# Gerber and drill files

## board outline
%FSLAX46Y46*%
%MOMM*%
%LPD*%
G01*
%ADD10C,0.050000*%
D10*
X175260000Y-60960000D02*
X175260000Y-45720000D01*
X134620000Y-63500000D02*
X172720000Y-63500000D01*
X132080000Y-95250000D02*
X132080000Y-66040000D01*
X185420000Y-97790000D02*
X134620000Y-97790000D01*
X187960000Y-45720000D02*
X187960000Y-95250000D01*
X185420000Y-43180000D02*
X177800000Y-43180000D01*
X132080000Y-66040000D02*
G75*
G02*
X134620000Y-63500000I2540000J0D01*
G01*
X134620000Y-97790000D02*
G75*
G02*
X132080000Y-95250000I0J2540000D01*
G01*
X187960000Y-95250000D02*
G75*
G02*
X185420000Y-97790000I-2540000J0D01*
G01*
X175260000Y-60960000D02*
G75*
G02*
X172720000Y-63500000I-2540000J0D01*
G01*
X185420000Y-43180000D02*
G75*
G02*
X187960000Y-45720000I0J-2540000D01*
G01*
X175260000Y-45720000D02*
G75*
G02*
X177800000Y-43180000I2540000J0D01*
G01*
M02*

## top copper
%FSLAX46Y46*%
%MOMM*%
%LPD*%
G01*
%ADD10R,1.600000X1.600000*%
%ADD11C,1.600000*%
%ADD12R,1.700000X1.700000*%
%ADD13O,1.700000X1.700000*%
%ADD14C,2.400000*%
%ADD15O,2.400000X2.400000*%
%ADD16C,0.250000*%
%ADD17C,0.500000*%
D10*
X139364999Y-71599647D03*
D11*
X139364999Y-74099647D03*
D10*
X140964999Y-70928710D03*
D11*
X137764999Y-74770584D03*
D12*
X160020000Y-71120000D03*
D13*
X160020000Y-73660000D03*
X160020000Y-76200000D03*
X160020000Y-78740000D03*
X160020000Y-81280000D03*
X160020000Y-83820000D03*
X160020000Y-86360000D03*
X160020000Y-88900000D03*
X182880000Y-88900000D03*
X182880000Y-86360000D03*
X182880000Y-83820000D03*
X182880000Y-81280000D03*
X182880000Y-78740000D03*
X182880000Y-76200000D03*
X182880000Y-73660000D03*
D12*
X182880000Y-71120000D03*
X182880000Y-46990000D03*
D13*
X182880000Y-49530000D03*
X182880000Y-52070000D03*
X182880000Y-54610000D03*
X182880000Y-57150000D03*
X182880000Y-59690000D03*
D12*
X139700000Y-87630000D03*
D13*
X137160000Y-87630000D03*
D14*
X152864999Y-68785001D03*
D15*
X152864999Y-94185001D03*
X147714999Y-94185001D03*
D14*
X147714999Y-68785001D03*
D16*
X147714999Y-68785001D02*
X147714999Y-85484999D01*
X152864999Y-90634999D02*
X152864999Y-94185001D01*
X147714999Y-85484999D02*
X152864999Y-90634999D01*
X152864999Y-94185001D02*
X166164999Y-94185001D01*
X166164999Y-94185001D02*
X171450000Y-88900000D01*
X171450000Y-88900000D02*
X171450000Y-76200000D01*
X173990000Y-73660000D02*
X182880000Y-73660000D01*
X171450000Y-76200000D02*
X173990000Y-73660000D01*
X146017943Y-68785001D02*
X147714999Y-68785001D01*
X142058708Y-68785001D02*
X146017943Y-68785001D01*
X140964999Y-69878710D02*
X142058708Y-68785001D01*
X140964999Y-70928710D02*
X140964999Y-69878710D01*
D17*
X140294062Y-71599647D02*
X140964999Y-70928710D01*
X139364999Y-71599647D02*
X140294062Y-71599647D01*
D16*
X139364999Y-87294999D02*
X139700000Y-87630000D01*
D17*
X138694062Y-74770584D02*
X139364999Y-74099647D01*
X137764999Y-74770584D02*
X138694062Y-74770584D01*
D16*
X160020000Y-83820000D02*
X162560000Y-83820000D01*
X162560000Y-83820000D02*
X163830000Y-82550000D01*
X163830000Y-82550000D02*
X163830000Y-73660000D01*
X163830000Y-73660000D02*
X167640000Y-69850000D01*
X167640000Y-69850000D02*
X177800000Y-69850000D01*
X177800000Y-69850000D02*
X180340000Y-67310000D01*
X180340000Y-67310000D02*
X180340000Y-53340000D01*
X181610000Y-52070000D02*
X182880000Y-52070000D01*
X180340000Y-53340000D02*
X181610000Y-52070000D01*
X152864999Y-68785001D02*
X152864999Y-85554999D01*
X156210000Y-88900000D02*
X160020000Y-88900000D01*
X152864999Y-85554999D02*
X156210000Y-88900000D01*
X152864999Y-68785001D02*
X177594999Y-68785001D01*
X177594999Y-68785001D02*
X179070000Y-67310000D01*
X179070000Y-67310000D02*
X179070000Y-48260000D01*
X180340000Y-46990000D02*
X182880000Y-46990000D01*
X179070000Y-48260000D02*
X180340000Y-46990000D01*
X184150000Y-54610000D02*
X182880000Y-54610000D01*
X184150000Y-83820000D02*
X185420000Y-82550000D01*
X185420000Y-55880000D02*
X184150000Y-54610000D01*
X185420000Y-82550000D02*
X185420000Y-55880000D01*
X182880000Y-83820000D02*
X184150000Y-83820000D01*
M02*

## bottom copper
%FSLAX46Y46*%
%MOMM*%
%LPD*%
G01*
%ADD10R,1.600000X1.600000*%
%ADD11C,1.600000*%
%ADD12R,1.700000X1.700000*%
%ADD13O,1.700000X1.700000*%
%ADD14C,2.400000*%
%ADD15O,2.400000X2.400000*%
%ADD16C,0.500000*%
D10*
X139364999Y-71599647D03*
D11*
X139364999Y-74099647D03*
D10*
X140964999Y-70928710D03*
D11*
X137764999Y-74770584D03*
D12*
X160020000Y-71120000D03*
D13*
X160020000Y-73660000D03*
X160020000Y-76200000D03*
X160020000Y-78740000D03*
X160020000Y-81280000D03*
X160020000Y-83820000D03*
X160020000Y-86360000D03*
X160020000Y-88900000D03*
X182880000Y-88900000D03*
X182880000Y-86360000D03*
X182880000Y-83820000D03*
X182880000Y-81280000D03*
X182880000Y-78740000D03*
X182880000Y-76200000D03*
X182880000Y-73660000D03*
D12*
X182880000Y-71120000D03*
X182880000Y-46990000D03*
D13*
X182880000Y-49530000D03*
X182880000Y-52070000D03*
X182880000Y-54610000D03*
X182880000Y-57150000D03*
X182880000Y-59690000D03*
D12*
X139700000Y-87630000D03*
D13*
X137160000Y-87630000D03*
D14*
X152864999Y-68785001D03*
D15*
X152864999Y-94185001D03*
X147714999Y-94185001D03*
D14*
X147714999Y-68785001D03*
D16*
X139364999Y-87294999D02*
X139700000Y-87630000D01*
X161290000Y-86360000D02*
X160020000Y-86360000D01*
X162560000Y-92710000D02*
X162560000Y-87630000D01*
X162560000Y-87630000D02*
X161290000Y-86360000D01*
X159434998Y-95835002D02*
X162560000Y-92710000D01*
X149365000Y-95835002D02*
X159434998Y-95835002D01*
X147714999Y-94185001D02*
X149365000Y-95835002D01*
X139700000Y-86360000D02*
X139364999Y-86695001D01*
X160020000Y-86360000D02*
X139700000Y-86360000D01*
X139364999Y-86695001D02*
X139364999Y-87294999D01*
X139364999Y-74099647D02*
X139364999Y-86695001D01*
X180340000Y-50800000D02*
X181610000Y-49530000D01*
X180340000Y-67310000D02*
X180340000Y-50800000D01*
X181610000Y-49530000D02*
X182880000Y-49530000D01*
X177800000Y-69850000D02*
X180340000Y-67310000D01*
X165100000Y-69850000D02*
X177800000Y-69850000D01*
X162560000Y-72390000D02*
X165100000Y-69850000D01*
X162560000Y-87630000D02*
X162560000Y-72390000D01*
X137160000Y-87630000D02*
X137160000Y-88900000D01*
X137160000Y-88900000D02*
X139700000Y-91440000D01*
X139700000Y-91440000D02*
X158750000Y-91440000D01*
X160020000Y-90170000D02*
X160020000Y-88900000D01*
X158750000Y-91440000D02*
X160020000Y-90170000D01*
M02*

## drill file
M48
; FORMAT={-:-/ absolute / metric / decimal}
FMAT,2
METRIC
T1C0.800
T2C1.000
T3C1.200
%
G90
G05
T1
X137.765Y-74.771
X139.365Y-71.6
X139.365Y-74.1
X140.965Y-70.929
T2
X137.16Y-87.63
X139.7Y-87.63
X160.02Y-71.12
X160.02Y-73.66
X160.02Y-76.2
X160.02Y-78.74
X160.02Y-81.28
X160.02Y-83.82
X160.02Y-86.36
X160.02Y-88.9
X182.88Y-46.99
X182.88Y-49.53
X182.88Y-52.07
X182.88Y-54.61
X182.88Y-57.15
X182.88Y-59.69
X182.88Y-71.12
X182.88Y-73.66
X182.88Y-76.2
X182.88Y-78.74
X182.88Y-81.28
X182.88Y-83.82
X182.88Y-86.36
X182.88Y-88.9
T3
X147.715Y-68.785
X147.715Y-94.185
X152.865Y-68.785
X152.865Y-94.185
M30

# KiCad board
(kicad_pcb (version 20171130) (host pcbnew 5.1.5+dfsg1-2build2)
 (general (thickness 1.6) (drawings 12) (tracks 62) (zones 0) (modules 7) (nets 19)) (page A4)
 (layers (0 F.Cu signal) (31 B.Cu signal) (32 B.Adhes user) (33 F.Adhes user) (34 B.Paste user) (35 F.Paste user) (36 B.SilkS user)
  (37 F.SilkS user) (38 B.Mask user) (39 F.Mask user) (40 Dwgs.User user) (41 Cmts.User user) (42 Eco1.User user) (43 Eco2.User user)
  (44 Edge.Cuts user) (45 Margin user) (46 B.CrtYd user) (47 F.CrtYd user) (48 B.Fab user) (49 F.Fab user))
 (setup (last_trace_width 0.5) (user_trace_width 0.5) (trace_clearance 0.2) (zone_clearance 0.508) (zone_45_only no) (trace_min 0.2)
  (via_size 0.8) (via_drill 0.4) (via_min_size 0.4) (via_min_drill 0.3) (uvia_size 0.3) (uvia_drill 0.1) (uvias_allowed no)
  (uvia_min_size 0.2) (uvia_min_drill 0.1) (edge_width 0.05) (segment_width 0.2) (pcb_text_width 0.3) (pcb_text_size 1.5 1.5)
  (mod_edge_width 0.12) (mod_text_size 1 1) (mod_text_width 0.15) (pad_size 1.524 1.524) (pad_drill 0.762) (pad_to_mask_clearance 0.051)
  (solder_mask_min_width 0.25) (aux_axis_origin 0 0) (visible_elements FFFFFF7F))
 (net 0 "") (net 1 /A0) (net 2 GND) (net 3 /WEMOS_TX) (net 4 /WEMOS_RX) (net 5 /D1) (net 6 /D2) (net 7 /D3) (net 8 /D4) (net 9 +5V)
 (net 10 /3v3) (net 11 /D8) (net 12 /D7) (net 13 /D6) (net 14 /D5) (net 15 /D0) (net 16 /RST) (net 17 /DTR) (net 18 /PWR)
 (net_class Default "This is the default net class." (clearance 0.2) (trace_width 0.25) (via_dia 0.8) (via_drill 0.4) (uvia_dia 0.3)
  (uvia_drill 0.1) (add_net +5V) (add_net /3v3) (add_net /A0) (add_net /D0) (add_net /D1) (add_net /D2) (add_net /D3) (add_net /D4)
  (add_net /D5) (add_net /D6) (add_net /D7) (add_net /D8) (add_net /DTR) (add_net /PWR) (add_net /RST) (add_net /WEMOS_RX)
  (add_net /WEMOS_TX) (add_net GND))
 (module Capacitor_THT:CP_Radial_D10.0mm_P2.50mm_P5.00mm (layer F.Cu) (at 139.364999 71.599647 270)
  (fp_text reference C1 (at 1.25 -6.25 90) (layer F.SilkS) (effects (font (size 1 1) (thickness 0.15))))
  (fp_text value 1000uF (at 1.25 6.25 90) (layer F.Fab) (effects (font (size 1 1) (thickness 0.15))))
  (pad 1 thru_hole rect (at 0 0 270) (size 1.6 1.6) (drill 0.8) (layers *.Cu *.Mask) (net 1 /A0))
  (pad 2 thru_hole circle (at 2.5 0 270) (size 1.6 1.6) (drill 0.8) (layers *.Cu *.Mask) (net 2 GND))
  (pad 1 thru_hole rect (at -0.670937 -1.6 270) (size 1.6 1.6) (drill 0.8) (layers *.Cu *.Mask) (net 1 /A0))
  (pad 2 thru_hole circle (at 3.170937 1.6 270) (size 1.6 1.6) (drill 0.8) (layers *.Cu *.Mask) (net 2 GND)))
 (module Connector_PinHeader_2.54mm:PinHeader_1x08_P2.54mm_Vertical (layer F.Cu) (at 160.02 71.12)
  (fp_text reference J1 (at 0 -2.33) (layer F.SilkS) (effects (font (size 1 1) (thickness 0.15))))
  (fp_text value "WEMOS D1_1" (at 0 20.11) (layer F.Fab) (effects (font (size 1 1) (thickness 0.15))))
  (pad 1 thru_hole rect (at 0 0) (size 1.7 1.7) (drill 1) (layers *.Cu *.Mask) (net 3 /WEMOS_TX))
  (pad 2 thru_hole oval (at 0 2.54) (size 1.7 1.7) (drill 1) (layers *.Cu *.Mask) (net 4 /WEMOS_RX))
  (pad 3 thru_hole oval (at 0 5.08) (size 1.7 1.7) (drill 1) (layers *.Cu *.Mask) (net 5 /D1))
  (pad 4 thru_hole oval (at 0 7.62) (size 1.7 1.7) (drill 1) (layers *.Cu *.Mask) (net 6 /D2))
  (pad 5 thru_hole oval (at 0 10.16) (size 1.7 1.7) (drill 1) (layers *.Cu *.Mask) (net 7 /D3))
  (pad 6 thru_hole oval (at 0 12.7) (size 1.7 1.7) (drill 1) (layers *.Cu *.Mask) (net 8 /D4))
  (pad 7 thru_hole oval (at 0 15.24) (size 1.7 1.7) (drill 1) (layers *.Cu *.Mask) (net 2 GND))
  (pad 8 thru_hole oval (at 0 17.78) (size 1.7 1.7) (drill 1) (layers *.Cu *.Mask) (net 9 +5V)))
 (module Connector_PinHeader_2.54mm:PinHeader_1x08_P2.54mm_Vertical (layer F.Cu) (at 182.88 71.12)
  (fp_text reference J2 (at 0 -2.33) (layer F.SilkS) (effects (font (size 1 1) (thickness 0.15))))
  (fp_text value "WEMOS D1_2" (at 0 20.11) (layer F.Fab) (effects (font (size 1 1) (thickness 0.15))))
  (pad 8 thru_hole oval (at 0 17.78) (size 1.7 1.7) (drill 1) (layers *.Cu *.Mask) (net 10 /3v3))
  (pad 7 thru_hole oval (at 0 15.24) (size 1.7 1.7) (drill 1) (layers *.Cu *.Mask) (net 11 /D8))
  (pad 6 thru_hole oval (at 0 12.7) (size 1.7 1.7) (drill 1) (layers *.Cu *.Mask) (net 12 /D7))
  (pad 5 thru_hole oval (at 0 10.16) (size 1.7 1.7) (drill 1) (layers *.Cu *.Mask) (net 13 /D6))
  (pad 4 thru_hole oval (at 0 7.62) (size 1.7 1.7) (drill 1) (layers *.Cu *.Mask) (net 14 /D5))
  (pad 3 thru_hole oval (at 0 5.08) (size 1.7 1.7) (drill 1) (layers *.Cu *.Mask) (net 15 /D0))
  (pad 2 thru_hole oval (at 0 2.54) (size 1.7 1.7) (drill 1) (layers *.Cu *.Mask) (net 1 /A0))
  (pad 1 thru_hole rect (at 0 0) (size 1.7 1.7) (drill 1) (layers *.Cu *.Mask) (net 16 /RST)))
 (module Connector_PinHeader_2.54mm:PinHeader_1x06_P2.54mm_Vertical (layer F.Cu) (at 182.88 46.99)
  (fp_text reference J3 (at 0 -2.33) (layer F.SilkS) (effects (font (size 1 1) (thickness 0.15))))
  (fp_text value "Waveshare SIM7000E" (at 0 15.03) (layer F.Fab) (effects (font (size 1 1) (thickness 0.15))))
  (pad 1 thru_hole rect (at 0 0) (size 1.7 1.7) (drill 1) (layers *.Cu *.Mask) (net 9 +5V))
  (pad 2 thru_hole oval (at 0 2.54) (size 1.7 1.7) (drill 1) (layers *.Cu *.Mask) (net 2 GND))
  (pad 3 thru_hole oval (at 0 5.08) (size 1.7 1.7) (drill 1) (layers *.Cu *.Mask) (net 8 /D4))
  (pad 4 thru_hole oval (at 0 7.62) (size 1.7 1.7) (drill 1) (layers *.Cu *.Mask) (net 12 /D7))
  (pad 5 thru_hole oval (at 0 10.16) (size 1.7 1.7) (drill 1) (layers *.Cu *.Mask) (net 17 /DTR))
  (pad 6 thru_hole oval (at 0 12.7) (size 1.7 1.7) (drill 1) (layers *.Cu *.Mask) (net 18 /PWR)))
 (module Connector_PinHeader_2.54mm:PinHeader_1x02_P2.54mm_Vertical (layer F.Cu) (at 139.7 87.63 270)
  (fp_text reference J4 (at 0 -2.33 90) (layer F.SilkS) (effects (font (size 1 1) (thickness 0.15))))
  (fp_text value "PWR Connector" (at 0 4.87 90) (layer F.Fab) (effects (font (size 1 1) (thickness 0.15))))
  (pad 1 thru_hole rect (at 0 0 270) (size 1.7 1.7) (drill 1) (layers *.Cu *.Mask) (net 2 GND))
  (pad 2 thru_hole oval (at 0 2.54 270) (size 1.7 1.7) (drill 1) (layers *.Cu *.Mask) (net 9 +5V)))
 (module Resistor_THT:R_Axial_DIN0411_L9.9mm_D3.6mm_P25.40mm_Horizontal (layer F.Cu) (at 152.864999 68.785001 270)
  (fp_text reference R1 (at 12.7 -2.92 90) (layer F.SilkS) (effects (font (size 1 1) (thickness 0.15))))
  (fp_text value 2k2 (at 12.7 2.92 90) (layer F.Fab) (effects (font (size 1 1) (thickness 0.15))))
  (pad 1 thru_hole circle (at 0 0 270) (size 2.4 2.4) (drill 1.2) (layers *.Cu *.Mask) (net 9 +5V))
  (pad 2 thru_hole oval (at 25.4 0 270) (size 2.4 2.4) (drill 1.2) (layers *.Cu *.Mask) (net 1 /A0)))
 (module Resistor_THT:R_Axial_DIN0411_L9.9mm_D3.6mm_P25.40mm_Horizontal (layer F.Cu) (at 147.714999 68.785001 270)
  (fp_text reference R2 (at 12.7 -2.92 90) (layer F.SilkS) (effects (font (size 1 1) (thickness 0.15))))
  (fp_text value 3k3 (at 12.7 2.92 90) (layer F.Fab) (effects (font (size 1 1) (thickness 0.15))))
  (pad 2 thru_hole oval (at 25.4 0 270) (size 2.4 2.4) (drill 1.2) (layers *.Cu *.Mask) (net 2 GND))
  (pad 1 thru_hole circle (at 0 0 270) (size 2.4 2.4) (drill 1.2) (layers *.Cu *.Mask) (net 1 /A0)))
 (gr_line (start 175.26 60.96) (end 175.26 45.72) (layer Edge.Cuts) (width 0.05))
 (gr_line (start 134.62 63.5) (end 172.72 63.5) (layer Edge.Cuts) (width 0.05))
 (gr_line (start 132.08 95.25) (end 132.08 66.04) (layer Edge.Cuts) (width 0.05))
 (gr_line (start 185.42 97.79) (end 134.62 97.79) (layer Edge.Cuts) (width 0.05))
 (gr_line (start 187.96 45.72) (end 187.96 95.25) (layer Edge.Cuts) (width 0.05))
 (gr_line (start 185.42 43.18) (end 177.8 43.18) (layer Edge.Cuts) (width 0.05))
 (gr_arc (start 134.62 66.04) (end 134.62 63.5) (angle -90) (layer Edge.Cuts) (width 0.05))
 (gr_arc (start 134.62 95.25) (end 132.08 95.25) (angle -90) (layer Edge.Cuts) (width 0.05))
 (gr_arc (start 185.42 95.25) (end 185.42 97.79) (angle -90) (layer Edge.Cuts) (width 0.05))
 (gr_arc (start 172.72 60.96) (end 172.72 63.5) (angle -90) (layer Edge.Cuts) (width 0.05))
 (gr_arc (start 185.42 45.72) (end 187.96 45.72) (angle -90) (layer Edge.Cuts) (width 0.05))
 (gr_arc (start 177.8 45.72) (end 177.8 43.18) (angle -90) (layer Edge.Cuts) (width 0.05))
 (segment (start 147.714999 68.785001) (end 147.714999 85.484999) (width 0.25) (layer F.Cu) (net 1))
 (segment (start 152.864999 90.634999) (end 152.864999 94.185001) (width 0.25) (layer F.Cu) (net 1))
 (segment (start 147.714999 85.484999) (end 152.864999 90.634999) (width 0.25) (layer F.Cu) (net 1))
 (segment (start 152.864999 94.185001) (end 166.164999 94.185001) (width 0.25) (layer F.Cu) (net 1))
 (segment (start 166.164999 94.185001) (end 171.45 88.9) (width 0.25) (layer F.Cu) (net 1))
 (segment (start 171.45 88.9) (end 171.45 76.2) (width 0.25) (layer F.Cu) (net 1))
 (segment (start 173.99 73.66) (end 182.88 73.66) (width 0.25) (layer F.Cu) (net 1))
 (segment (start 171.45 76.2) (end 173.99 73.66) (width 0.25) (layer F.Cu) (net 1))
 (segment (start 146.017943 68.785001) (end 147.714999 68.785001) (width 0.25) (layer F.Cu) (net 1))
 (segment (start 142.058708 68.785001) (end 146.017943 68.785001) (width 0.25) (layer F.Cu) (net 1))
 (segment (start 140.964999 69.87871) (end 142.058708 68.785001) (width 0.25) (layer F.Cu) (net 1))
 (segment (start 140.964999 70.92871) (end 140.964999 69.87871) (width 0.25) (layer F.Cu) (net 1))
 (segment (start 140.294062 71.599647) (end 140.964999 70.92871) (width 0.5) (layer F.Cu) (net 1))
 (segment (start 139.364999 71.599647) (end 140.294062 71.599647) (width 0.5) (layer F.Cu) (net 1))
 (segment (start 139.364999 87.294999) (end 139.7 87.63) (width 0.25) (layer F.Cu) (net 2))
 (segment (start 139.364999 87.294999) (end 139.7 87.63) (width 0.5) (layer B.Cu) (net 2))
 (segment (start 161.29 86.36) (end 160.02 86.36) (width 0.5) (layer B.Cu) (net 2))
 (segment (start 162.56 92.71) (end 162.56 87.63) (width 0.5) (layer B.Cu) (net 2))
 (segment (start 162.56 87.63) (end 161.29 86.36) (width 0.5) (layer B.Cu) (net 2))
 (segment (start 159.434998 95.835002) (end 162.56 92.71) (width 0.5) (layer B.Cu) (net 2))
 (segment (start 149.365 95.835002) (end 159.434998 95.835002) (width 0.5) (layer B.Cu) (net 2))
 (segment (start 147.714999 94.185001) (end 149.365 95.835002) (width 0.5) (layer B.Cu) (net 2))
 (segment (start 139.7 86.36) (end 139.364999 86.695001) (width 0.5) (layer B.Cu) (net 2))
 (segment (start 160.02 86.36) (end 139.7 86.36) (width 0.5) (layer B.Cu) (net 2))
 (segment (start 139.364999 86.695001) (end 139.364999 87.294999) (width 0.5) (layer B.Cu) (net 2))
 (segment (start 139.364999 74.099647) (end 139.364999 86.695001) (width 0.5) (layer B.Cu) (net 2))
 (segment (start 180.34 50.8) (end 181.61 49.53) (width 0.5) (layer B.Cu) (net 2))
 (segment (start 180.34 67.31) (end 180.34 50.8) (width 0.5) (layer B.Cu) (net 2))
 (segment (start 181.61 49.53) (end 182.88 49.53) (width 0.5) (layer B.Cu) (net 2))
 (segment (start 177.8 69.85) (end 180.34 67.31) (width 0.5) (layer B.Cu) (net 2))
 (segment (start 165.1 69.85) (end 177.8 69.85) (width 0.5) (layer B.Cu) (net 2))
 (segment (start 162.56 72.39) (end 165.1 69.85) (width 0.5) (layer B.Cu) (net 2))
 (segment (start 162.56 87.63) (end 162.56 72.39) (width 0.5) (layer B.Cu) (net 2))
 (segment (start 138.694062 74.770584) (end 139.364999 74.099647) (width 0.5) (layer F.Cu) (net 2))
 (segment (start 137.764999 74.770584) (end 138.694062 74.770584) (width 0.5) (layer F.Cu) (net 2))
 (segment (start 160.02 83.82) (end 162.56 83.82) (width 0.25) (layer F.Cu) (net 8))
 (segment (start 162.56 83.82) (end 163.83 82.55) (width 0.25) (layer F.Cu) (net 8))
 (segment (start 163.83 82.55) (end 163.83 73.66) (width 0.25) (layer F.Cu) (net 8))
 (segment (start 163.83 73.66) (end 167.64 69.85) (width 0.25) (layer F.Cu) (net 8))
 (segment (start 167.64 69.85) (end 177.8 69.85) (width 0.25) (layer F.Cu) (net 8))
 (segment (start 177.8 69.85) (end 180.34 67.31) (width 0.25) (layer F.Cu) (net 8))
 (segment (start 180.34 67.31) (end 180.34 53.34) (width 0.25) (layer F.Cu) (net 8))
 (segment (start 181.61 52.07) (end 182.88 52.07) (width 0.25) (layer F.Cu) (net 8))
 (segment (start 180.34 53.34) (end 181.61 52.07) (width 0.25) (layer F.Cu) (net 8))
 (segment (start 152.864999 68.785001) (end 152.864999 85.554999) (width 0.25) (layer F.Cu) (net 9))
 (segment (start 156.21 88.9) (end 160.02 88.9) (width 0.25) (layer F.Cu) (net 9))
 (segment (start 152.864999 85.554999) (end 156.21 88.9) (width 0.25) (layer F.Cu) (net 9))
 (segment (start 137.16 87.63) (end 137.16 88.9) (width 0.5) (layer B.Cu) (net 9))
 (segment (start 137.16 88.9) (end 139.7 91.44) (width 0.5) (layer B.Cu) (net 9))
 (segment (start 139.7 91.44) (end 158.75 91.44) (width 0.5) (layer B.Cu) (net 9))
 (segment (start 160.02 90.17) (end 160.02 88.9) (width 0.5) (layer B.Cu) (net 9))
 (segment (start 158.75 91.44) (end 160.02 90.17) (width 0.5) (layer B.Cu) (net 9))
 (segment (start 152.864999 68.785001) (end 177.594999 68.785001) (width 0.25) (layer F.Cu) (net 9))
 (segment (start 177.594999 68.785001) (end 179.07 67.31) (width 0.25) (layer F.Cu) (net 9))
 (segment (start 179.07 67.31) (end 179.07 48.26) (width 0.25) (layer F.Cu) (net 9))
 (segment (start 180.34 46.99) (end 182.88 46.99) (width 0.25) (layer F.Cu) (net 9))
 (segment (start 179.07 48.26) (end 180.34 46.99) (width 0.25) (layer F.Cu) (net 9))
 (segment (start 184.15 54.61) (end 182.88 54.61) (width 0.25) (layer F.Cu) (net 12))
 (segment (start 184.15 83.82) (end 185.42 82.55) (width 0.25) (layer F.Cu) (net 12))
 (segment (start 185.42 55.88) (end 184.15 54.61) (width 0.25) (layer F.Cu) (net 12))
 (segment (start 185.42 82.55) (end 185.42 55.88) (width 0.25) (layer F.Cu) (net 12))
 (segment (start 182.88 83.82) (end 184.15 83.82) (width 0.25) (layer F.Cu) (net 12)))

